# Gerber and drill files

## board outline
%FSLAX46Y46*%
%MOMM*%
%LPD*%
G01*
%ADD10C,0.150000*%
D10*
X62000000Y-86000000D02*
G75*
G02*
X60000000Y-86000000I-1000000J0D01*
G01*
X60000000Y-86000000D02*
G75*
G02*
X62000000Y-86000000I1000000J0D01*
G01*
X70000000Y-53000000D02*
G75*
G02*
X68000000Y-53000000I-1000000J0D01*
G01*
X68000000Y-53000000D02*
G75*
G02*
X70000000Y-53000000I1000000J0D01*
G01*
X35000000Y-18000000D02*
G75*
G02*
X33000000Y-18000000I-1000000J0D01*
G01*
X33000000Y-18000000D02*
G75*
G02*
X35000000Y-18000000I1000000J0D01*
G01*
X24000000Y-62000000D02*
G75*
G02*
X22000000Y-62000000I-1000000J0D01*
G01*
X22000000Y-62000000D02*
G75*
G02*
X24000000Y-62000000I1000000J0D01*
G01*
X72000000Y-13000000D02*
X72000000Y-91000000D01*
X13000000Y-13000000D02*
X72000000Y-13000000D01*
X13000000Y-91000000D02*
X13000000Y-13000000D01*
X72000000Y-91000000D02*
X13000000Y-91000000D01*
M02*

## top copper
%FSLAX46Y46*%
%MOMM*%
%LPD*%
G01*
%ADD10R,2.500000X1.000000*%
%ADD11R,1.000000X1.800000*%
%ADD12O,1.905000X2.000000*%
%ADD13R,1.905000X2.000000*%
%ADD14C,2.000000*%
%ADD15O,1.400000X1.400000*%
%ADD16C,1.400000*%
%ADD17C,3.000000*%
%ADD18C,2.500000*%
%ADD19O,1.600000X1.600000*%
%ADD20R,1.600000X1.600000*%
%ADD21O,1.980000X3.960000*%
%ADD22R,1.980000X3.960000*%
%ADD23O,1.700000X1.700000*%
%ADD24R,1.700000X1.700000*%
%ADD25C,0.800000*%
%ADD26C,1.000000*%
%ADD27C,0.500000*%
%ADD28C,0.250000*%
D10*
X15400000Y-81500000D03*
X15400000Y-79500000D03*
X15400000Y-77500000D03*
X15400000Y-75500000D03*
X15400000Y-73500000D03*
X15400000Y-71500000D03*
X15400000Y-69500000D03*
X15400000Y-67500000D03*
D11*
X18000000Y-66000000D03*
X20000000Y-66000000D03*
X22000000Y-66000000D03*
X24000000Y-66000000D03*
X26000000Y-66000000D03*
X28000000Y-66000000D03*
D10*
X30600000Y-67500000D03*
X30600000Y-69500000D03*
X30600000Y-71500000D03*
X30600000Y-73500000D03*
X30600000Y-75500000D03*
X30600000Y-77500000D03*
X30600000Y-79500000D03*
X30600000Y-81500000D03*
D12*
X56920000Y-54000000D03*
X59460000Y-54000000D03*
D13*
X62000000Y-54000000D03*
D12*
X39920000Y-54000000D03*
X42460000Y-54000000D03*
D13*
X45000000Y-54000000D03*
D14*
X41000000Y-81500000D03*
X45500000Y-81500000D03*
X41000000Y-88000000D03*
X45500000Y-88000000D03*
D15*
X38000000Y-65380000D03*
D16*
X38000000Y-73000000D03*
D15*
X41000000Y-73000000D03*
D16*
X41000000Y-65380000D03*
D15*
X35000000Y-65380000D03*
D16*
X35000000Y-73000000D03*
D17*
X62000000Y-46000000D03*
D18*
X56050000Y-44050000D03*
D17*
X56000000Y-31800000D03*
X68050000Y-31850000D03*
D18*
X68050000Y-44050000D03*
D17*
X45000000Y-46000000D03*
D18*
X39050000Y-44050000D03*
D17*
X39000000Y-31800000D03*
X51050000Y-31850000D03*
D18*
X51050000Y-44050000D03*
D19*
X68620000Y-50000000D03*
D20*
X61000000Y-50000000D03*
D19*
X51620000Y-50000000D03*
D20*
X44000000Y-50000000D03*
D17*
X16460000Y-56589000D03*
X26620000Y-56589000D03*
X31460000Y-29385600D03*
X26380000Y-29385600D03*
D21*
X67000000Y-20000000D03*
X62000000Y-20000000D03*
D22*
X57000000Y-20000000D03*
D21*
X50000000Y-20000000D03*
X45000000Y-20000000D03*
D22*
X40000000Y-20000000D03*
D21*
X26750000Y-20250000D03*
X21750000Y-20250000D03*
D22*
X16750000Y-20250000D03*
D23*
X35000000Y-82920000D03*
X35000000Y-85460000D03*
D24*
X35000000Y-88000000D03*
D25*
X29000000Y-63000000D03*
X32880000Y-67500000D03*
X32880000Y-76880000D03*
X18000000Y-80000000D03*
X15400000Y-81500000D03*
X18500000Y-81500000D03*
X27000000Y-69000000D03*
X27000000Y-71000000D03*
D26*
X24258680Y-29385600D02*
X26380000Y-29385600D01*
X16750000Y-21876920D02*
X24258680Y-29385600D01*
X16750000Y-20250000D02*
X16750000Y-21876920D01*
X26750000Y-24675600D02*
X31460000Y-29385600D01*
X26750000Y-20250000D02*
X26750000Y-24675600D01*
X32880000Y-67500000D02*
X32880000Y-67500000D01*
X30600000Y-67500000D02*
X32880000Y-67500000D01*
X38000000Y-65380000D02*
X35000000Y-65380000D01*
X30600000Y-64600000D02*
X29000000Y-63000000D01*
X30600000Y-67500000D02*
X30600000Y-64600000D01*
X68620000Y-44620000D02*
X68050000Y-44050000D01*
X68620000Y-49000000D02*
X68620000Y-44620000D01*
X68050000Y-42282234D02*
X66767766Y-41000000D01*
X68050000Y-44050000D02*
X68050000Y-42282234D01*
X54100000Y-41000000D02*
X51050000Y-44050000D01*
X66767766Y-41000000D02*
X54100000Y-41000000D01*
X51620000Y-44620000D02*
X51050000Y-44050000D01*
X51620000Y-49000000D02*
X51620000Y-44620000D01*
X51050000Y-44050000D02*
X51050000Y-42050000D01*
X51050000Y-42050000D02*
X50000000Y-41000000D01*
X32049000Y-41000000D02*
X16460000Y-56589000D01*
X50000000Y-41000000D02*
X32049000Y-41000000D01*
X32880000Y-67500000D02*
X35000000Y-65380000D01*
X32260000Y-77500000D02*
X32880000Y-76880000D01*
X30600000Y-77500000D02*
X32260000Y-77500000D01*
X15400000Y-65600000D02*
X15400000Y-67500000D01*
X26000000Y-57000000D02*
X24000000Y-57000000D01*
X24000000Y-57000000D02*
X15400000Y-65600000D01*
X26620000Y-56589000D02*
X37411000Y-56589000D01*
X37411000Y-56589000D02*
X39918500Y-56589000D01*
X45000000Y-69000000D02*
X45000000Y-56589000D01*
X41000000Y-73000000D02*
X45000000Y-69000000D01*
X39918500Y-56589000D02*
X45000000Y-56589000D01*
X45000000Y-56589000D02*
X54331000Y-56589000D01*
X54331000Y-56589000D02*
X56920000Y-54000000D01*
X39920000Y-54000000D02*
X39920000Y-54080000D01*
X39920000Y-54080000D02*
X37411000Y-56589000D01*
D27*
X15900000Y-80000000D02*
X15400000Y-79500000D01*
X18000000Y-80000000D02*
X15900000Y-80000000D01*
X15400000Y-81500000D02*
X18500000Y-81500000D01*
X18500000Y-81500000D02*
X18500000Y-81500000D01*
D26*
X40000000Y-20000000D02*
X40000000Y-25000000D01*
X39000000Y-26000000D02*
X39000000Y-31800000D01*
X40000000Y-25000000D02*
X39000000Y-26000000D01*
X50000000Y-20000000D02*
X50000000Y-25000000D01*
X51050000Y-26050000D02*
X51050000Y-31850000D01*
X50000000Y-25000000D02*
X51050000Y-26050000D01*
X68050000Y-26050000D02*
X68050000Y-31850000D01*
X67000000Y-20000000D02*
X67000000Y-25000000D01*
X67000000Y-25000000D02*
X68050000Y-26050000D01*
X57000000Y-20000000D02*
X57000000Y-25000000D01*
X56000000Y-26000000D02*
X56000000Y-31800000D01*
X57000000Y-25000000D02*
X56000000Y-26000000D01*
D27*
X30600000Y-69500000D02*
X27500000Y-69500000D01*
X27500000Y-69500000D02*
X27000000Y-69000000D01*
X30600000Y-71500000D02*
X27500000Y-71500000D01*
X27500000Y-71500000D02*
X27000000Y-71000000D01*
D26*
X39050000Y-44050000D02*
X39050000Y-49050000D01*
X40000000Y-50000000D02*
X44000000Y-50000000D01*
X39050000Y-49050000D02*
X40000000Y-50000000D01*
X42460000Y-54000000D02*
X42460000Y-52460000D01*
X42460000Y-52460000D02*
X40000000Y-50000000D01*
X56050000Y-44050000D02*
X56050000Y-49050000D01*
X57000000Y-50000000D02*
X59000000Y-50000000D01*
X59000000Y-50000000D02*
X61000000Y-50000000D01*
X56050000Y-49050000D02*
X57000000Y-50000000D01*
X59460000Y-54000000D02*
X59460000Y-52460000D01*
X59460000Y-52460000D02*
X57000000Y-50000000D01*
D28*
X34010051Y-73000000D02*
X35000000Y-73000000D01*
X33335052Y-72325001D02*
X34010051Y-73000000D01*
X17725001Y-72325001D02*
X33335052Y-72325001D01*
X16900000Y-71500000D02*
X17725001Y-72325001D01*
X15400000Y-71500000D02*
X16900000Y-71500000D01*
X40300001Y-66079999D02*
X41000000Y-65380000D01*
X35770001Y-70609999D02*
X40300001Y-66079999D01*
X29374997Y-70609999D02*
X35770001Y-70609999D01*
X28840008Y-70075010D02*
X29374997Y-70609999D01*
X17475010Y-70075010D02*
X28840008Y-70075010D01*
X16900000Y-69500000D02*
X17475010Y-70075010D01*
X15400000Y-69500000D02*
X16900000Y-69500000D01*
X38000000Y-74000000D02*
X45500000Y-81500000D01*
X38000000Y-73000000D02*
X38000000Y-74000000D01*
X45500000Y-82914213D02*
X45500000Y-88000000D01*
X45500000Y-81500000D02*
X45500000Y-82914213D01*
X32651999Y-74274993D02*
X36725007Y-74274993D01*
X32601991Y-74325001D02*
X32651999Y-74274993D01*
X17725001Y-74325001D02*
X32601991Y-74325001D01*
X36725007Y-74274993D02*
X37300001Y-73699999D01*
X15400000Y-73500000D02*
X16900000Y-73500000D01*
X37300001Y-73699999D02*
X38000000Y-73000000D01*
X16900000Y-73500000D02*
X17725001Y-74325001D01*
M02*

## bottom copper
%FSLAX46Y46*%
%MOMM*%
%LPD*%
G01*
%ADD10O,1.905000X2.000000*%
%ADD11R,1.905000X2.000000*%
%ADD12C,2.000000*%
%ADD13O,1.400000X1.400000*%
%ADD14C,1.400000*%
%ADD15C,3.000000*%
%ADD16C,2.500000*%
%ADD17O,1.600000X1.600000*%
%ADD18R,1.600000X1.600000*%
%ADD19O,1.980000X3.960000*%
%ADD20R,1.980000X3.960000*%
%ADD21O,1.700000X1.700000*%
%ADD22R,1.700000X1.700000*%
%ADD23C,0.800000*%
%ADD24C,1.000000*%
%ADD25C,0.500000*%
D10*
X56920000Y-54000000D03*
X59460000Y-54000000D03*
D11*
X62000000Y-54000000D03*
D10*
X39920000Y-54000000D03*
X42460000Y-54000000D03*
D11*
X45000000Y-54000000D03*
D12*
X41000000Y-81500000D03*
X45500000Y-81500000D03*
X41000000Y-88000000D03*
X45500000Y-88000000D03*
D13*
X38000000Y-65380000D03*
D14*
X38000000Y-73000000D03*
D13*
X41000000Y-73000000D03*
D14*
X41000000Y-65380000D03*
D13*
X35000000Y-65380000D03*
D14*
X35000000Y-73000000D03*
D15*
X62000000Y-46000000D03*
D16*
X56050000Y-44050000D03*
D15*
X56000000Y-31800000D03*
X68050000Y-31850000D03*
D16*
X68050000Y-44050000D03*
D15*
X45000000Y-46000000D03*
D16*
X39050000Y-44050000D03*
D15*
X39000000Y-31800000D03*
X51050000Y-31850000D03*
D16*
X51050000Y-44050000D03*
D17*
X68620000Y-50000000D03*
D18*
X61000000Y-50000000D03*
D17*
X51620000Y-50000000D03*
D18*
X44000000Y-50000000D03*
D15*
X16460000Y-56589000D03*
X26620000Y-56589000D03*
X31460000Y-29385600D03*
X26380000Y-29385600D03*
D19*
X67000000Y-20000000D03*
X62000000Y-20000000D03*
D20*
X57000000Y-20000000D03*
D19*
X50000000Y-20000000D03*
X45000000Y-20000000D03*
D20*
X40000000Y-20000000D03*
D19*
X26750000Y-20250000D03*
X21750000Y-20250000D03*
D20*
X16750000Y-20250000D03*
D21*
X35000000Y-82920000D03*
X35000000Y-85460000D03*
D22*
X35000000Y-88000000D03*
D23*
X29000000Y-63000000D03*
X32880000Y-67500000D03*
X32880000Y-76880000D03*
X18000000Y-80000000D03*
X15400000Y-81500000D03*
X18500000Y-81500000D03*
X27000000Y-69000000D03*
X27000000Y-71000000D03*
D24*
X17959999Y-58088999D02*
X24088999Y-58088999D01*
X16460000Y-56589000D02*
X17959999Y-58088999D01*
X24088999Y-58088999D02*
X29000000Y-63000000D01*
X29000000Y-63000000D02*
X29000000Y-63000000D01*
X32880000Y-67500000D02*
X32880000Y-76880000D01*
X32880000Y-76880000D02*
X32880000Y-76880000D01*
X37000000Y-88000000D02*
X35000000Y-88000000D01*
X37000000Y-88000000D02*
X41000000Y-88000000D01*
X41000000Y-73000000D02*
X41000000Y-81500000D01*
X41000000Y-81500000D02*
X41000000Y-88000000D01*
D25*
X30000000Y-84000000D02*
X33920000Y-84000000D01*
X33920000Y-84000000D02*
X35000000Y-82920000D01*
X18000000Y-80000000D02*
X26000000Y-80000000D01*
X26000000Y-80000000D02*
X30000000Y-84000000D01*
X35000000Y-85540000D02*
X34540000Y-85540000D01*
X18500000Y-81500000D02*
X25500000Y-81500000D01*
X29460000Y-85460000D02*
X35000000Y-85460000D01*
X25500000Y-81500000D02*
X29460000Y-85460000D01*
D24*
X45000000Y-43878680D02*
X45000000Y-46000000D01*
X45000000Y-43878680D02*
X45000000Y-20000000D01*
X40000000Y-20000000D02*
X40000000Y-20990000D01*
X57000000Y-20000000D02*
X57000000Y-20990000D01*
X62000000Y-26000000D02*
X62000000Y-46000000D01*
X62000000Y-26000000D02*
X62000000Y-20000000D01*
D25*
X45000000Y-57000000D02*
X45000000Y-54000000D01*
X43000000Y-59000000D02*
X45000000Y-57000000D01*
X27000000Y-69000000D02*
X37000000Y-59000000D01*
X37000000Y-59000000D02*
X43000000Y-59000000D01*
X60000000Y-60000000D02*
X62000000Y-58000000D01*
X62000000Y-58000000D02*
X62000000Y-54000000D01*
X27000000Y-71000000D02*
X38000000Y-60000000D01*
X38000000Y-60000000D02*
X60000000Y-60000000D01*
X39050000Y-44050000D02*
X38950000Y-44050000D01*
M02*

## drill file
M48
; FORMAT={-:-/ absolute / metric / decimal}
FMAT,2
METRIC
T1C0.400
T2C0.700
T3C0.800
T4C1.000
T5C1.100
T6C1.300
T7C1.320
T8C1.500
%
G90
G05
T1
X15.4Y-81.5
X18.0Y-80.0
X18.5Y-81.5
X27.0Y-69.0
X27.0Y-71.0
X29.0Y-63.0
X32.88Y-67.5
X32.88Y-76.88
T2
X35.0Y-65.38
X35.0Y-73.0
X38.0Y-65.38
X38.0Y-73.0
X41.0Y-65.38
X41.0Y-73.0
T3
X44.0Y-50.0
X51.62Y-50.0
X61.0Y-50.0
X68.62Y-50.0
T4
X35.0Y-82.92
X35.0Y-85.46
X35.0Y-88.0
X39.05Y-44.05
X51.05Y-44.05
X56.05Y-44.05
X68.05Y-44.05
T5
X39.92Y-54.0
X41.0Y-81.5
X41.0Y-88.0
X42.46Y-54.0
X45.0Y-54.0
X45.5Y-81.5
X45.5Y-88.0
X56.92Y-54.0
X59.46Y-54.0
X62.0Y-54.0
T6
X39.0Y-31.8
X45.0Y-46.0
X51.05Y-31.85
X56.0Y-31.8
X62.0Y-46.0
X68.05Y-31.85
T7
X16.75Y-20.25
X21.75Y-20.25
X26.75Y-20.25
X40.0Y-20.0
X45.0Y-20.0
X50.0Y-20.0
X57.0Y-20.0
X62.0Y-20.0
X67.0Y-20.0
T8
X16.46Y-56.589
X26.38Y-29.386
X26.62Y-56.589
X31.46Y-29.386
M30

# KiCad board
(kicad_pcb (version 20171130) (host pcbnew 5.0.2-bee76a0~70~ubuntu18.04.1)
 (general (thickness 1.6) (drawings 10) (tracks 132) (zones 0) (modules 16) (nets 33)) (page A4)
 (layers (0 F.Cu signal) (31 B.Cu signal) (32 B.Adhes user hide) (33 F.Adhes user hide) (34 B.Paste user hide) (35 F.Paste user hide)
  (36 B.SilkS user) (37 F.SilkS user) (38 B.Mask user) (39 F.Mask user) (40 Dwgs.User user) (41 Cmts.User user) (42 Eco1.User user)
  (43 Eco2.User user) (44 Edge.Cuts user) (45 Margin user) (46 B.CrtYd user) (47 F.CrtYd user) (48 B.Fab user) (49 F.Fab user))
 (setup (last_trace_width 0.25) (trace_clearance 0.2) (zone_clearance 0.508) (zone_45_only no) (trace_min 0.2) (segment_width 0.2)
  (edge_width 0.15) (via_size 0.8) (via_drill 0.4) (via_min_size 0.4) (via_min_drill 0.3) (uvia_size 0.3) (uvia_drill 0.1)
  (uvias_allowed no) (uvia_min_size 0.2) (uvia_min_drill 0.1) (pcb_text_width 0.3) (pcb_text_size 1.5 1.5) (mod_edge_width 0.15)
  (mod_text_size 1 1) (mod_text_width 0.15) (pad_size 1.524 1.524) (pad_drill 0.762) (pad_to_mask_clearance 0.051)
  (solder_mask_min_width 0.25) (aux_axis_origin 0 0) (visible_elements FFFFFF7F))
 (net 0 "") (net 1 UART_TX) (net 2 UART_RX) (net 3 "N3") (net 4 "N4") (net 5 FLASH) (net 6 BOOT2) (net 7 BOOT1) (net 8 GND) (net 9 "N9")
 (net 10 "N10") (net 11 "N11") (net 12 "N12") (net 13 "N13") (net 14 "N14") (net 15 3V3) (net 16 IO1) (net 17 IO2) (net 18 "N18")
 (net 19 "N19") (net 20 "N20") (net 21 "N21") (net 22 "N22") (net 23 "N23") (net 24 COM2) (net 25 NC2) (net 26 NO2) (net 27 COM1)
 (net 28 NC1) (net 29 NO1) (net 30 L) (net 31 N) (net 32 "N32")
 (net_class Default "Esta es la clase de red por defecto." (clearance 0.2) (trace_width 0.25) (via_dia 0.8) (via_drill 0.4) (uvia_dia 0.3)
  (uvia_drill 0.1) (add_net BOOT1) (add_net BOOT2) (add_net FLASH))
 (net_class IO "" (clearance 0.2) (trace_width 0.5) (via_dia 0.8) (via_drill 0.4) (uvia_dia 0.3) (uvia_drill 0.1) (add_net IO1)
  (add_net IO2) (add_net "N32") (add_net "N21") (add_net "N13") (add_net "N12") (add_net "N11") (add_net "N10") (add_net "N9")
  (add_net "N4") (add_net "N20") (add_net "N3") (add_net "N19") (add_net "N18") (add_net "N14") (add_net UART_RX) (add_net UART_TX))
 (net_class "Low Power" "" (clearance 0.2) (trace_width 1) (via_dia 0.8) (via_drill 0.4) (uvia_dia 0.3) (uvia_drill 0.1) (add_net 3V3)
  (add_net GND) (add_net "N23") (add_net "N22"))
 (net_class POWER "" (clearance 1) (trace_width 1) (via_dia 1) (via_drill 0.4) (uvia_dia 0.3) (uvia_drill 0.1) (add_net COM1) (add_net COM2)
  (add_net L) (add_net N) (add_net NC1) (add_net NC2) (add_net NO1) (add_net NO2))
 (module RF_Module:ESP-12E (layer F.Cu) (at 23 78 180)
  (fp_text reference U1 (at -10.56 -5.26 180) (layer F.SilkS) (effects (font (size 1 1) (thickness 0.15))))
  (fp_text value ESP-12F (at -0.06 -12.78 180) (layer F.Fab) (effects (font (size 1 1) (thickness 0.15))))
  (pad 22 smd rect (at 7.6 -3.5 180) (size 2.5 1) (layers F.Cu F.Paste F.Mask) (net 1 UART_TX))
  (pad 21 smd rect (at 7.6 -1.5 180) (size 2.5 1) (layers F.Cu F.Paste F.Mask) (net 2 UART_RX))
  (pad 20 smd rect (at 7.6 0.5 180) (size 2.5 1) (layers F.Cu F.Paste F.Mask) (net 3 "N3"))
  (pad 19 smd rect (at 7.6 2.5 180) (size 2.5 1) (layers F.Cu F.Paste F.Mask) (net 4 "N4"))
  (pad 18 smd rect (at 7.6 4.5 180) (size 2.5 1) (layers F.Cu F.Paste F.Mask) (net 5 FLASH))
  (pad 17 smd rect (at 7.6 6.5 180) (size 2.5 1) (layers F.Cu F.Paste F.Mask) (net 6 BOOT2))
  (pad 16 smd rect (at 7.6 8.5 180) (size 2.5 1) (layers F.Cu F.Paste F.Mask) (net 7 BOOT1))
  (pad 15 smd rect (at 7.6 10.5 180) (size 2.5 1) (layers F.Cu F.Paste F.Mask) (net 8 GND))
  (pad 14 smd rect (at 5 12 180) (size 1 1.8) (layers F.Cu F.Paste F.Mask) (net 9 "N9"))
  (pad 13 smd rect (at 3 12 180) (size 1 1.8) (layers F.Cu F.Paste F.Mask) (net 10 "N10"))
  (pad 12 smd rect (at 1 12 180) (size 1 1.8) (layers F.Cu F.Paste F.Mask) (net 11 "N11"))
  (pad 11 smd rect (at -1 12 180) (size 1 1.8) (layers F.Cu F.Paste F.Mask) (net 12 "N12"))
  (pad 10 smd rect (at -3 12 180) (size 1 1.8) (layers F.Cu F.Paste F.Mask) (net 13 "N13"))
  (pad 9 smd rect (at -5 12 180) (size 1 1.8) (layers F.Cu F.Paste F.Mask) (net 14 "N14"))
  (pad 8 smd rect (at -7.6 10.5 180) (size 2.5 1) (layers F.Cu F.Paste F.Mask) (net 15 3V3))
  (pad 7 smd rect (at -7.6 8.5 180) (size 2.5 1) (layers F.Cu F.Paste F.Mask) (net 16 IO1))
  (pad 6 smd rect (at -7.6 6.5 180) (size 2.5 1) (layers F.Cu F.Paste F.Mask) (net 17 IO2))
  (pad 5 smd rect (at -7.6 4.5 180) (size 2.5 1) (layers F.Cu F.Paste F.Mask) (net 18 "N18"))
  (pad 4 smd rect (at -7.6 2.5 180) (size 2.5 1) (layers F.Cu F.Paste F.Mask) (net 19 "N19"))
  (pad 3 smd rect (at -7.6 0.5 180) (size 2.5 1) (layers F.Cu F.Paste F.Mask) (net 15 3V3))
  (pad 2 smd rect (at -7.6 -1.5 180) (size 2.5 1) (layers F.Cu F.Paste F.Mask) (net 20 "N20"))
  (pad 1 smd rect (at -7.6 -3.5 180) (size 2.5 1) (layers F.Cu F.Paste F.Mask) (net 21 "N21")))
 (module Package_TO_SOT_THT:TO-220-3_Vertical (layer F.Cu) (at 62 54 180)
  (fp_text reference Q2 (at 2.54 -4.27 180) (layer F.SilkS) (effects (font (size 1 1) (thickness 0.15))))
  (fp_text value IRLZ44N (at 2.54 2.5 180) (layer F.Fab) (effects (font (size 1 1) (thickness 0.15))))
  (pad 3 thru_hole oval (at 5.08 0 180) (size 1.905 2) (drill 1.1) (layers *.Cu *.Mask) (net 8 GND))
  (pad 2 thru_hole oval (at 2.54 0 180) (size 1.905 2) (drill 1.1) (layers *.Cu *.Mask) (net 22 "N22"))
  (pad 1 thru_hole rect (at 0 0 180) (size 1.905 2) (drill 1.1) (layers *.Cu *.Mask) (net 17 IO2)))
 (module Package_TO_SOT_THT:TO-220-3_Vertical (layer F.Cu) (at 45 54 180)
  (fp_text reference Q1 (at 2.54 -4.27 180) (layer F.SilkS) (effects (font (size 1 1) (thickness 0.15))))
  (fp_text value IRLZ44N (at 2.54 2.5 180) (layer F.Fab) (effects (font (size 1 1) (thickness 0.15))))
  (pad 3 thru_hole oval (at 5.08 0 180) (size 1.905 2) (drill 1.1) (layers *.Cu *.Mask) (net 8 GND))
  (pad 2 thru_hole oval (at 2.54 0 180) (size 1.905 2) (drill 1.1) (layers *.Cu *.Mask) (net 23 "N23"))
  (pad 1 thru_hole rect (at 0 0 180) (size 1.905 2) (drill 1.1) (layers *.Cu *.Mask) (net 16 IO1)))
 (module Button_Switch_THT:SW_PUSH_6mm (layer F.Cu) (at 41 88 90)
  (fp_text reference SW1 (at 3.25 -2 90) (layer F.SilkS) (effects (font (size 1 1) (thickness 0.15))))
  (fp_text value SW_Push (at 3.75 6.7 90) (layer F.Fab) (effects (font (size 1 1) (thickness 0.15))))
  (pad 1 thru_hole circle (at 6.5 0 180) (size 2 2) (drill 1.1) (layers *.Cu *.Mask) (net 8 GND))
  (pad 2 thru_hole circle (at 6.5 4.5 180) (size 2 2) (drill 1.1) (layers *.Cu *.Mask) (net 5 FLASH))
  (pad 1 thru_hole circle (at 0 0 180) (size 2 2) (drill 1.1) (layers *.Cu *.Mask) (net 8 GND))
  (pad 2 thru_hole circle (at 0 4.5 180) (size 2 2) (drill 1.1) (layers *.Cu *.Mask) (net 5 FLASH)))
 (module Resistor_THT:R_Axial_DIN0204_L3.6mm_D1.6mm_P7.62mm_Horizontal (layer F.Cu) (at 38 73 90)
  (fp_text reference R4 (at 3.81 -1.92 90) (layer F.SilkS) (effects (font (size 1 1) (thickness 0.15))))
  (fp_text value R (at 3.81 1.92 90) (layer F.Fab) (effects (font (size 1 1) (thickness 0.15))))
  (pad 2 thru_hole oval (at 7.62 0 90) (size 1.4 1.4) (drill 0.7) (layers *.Cu *.Mask) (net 15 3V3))
  (pad 1 thru_hole circle (at 0 0 90) (size 1.4 1.4) (drill 0.7) (layers *.Cu *.Mask) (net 5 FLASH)))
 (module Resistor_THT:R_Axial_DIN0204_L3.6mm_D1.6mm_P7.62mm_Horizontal (layer F.Cu) (at 41 65.38 270)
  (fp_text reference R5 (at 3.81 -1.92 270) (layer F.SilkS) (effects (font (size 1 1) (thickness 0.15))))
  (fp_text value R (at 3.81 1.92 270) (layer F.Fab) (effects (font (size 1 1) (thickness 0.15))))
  (pad 2 thru_hole oval (at 7.62 0 270) (size 1.4 1.4) (drill 0.7) (layers *.Cu *.Mask) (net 8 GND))
  (pad 1 thru_hole circle (at 0 0 270) (size 1.4 1.4) (drill 0.7) (layers *.Cu *.Mask) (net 7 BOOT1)))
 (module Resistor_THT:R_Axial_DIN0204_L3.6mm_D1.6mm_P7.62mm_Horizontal (layer F.Cu) (at 35 73 90)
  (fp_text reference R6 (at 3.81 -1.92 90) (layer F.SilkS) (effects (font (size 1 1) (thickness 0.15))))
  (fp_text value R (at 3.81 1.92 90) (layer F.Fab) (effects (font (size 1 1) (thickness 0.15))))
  (pad 2 thru_hole oval (at 7.62 0 90) (size 1.4 1.4) (drill 0.7) (layers *.Cu *.Mask) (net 15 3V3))
  (pad 1 thru_hole circle (at 0 0 90) (size 1.4 1.4) (drill 0.7) (layers *.Cu *.Mask) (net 6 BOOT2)))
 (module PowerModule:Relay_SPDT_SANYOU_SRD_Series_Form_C (layer F.Cu) (at 62 46 90)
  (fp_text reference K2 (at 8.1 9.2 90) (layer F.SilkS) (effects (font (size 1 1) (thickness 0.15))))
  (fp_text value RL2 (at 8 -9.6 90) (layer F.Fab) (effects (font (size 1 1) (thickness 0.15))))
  (pad 5 thru_hole circle (at 0 0 180) (size 3 3) (drill 1.3) (layers *.Cu *.Mask) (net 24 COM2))
  (pad 4 thru_hole circle (at 1.95 -5.95 180) (size 2.5 2.5) (drill 1) (layers *.Cu *.Mask) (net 22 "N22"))
  (pad 2 thru_hole circle (at 14.2 -6 180) (size 3 3) (drill 1.3) (layers *.Cu *.Mask) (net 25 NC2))
  (pad 1 thru_hole circle (at 14.15 6.05 180) (size 3 3) (drill 1.3) (layers *.Cu *.Mask) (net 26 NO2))
  (pad 3 thru_hole circle (at 1.95 6.05 180) (size 2.5 2.5) (drill 1) (layers *.Cu *.Mask) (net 15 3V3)))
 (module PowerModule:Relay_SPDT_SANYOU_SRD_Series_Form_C (layer F.Cu) (at 45 46 90)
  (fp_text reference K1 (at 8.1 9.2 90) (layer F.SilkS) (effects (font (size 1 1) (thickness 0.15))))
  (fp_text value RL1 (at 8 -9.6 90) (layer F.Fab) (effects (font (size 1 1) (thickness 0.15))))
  (pad 5 thru_hole circle (at 0 0 180) (size 3 3) (drill 1.3) (layers *.Cu *.Mask) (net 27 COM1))
  (pad 4 thru_hole circle (at 1.95 -5.95 180) (size 2.5 2.5) (drill 1) (layers *.Cu *.Mask) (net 23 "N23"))
  (pad 2 thru_hole circle (at 14.2 -6 180) (size 3 3) (drill 1.3) (layers *.Cu *.Mask) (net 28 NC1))
  (pad 1 thru_hole circle (at 14.15 6.05 180) (size 3 3) (drill 1.3) (layers *.Cu *.Mask) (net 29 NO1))
  (pad 3 thru_hole circle (at 1.95 6.05 180) (size 2.5 2.5) (drill 1) (layers *.Cu *.Mask) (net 15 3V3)))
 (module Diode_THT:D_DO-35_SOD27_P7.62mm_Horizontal (layer F.Cu) (at 61 50)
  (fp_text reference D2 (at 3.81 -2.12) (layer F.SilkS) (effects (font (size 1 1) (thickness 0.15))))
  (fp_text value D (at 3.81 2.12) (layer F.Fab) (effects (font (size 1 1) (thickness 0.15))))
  (pad 2 thru_hole oval (at 7.62 0) (size 1.6 1.6) (drill 0.8) (layers *.Cu *.Mask) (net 15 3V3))
  (pad 1 thru_hole rect (at 0 0) (size 1.6 1.6) (drill 0.8) (layers *.Cu *.Mask) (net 22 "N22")))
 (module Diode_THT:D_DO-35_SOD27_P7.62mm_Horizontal (layer F.Cu) (at 44 50)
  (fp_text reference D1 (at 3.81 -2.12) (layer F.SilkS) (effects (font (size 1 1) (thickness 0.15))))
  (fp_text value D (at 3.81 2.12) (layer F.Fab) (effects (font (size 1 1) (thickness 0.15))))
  (pad 2 thru_hole oval (at 7.62 0) (size 1.6 1.6) (drill 0.8) (layers *.Cu *.Mask) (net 15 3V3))
  (pad 1 thru_hole rect (at 0 0) (size 1.6 1.6) (drill 0.8) (layers *.Cu *.Mask) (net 23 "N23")))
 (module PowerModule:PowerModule (layer F.Cu) (at 24 43 270)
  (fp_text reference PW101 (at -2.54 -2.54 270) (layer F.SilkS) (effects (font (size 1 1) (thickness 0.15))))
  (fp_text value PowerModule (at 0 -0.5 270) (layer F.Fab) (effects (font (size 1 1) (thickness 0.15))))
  (pad 4 thru_hole circle (at 13.589 7.54 270) (size 3 3) (drill 1.5) (layers *.Cu *.Mask) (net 15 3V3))
  (pad 3 thru_hole circle (at 13.589 -2.62 270) (size 3 3) (drill 1.5) (layers *.Cu *.Mask) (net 8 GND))
  (pad 2 thru_hole circle (at -13.6144 -7.46 270) (size 3 3) (drill 1.5) (layers *.Cu *.Mask) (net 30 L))
  (pad 1 thru_hole circle (at -13.6144 -2.38 270) (size 3 3) (drill 1.5) (layers *.Cu *.Mask) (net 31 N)))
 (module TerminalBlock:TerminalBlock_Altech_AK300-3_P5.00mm (layer F.Cu) (at 57 20)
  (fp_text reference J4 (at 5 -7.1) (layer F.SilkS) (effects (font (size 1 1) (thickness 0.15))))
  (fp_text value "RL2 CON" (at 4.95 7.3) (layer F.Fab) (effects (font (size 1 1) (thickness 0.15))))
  (pad 3 thru_hole oval (at 10 0) (size 1.98 3.96) (drill 1.32) (layers *.Cu *.Mask) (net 26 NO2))
  (pad 2 thru_hole oval (at 5 0) (size 1.98 3.96) (drill 1.32) (layers *.Cu *.Mask) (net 24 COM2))
  (pad 1 thru_hole rect (at 0 0) (size 1.98 3.96) (drill 1.32) (layers *.Cu *.Mask) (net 25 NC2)))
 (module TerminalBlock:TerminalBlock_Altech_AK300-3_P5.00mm (layer F.Cu) (at 40 20)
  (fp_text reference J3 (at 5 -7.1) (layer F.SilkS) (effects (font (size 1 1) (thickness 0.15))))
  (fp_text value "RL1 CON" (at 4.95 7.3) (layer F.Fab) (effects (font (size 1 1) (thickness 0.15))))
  (pad 3 thru_hole oval (at 10 0) (size 1.98 3.96) (drill 1.32) (layers *.Cu *.Mask) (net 29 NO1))
  (pad 2 thru_hole oval (at 5 0) (size 1.98 3.96) (drill 1.32) (layers *.Cu *.Mask) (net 27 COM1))
  (pad 1 thru_hole rect (at 0 0) (size 1.98 3.96) (drill 1.32) (layers *.Cu *.Mask) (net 28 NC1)))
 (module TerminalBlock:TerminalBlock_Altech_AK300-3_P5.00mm (layer F.Cu) (at 16.75 20.25)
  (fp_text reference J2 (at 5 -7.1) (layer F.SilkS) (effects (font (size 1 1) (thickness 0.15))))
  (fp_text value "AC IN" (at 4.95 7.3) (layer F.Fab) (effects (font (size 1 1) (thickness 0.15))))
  (pad 3 thru_hole oval (at 10 0) (size 1.98 3.96) (drill 1.32) (layers *.Cu *.Mask) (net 30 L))
  (pad 2 thru_hole oval (at 5 0) (size 1.98 3.96) (drill 1.32) (layers *.Cu *.Mask) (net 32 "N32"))
  (pad 1 thru_hole rect (at 0 0) (size 1.98 3.96) (drill 1.32) (layers *.Cu *.Mask) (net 31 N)))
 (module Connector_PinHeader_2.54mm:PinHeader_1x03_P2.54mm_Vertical (layer F.Cu) (at 35 88 180)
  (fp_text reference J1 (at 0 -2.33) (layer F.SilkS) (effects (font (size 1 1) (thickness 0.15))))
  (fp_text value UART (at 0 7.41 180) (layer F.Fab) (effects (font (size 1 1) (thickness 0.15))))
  (pad 3 thru_hole oval (at 0 5.08 180) (size 1.7 1.7) (drill 1) (layers *.Cu *.Mask) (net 2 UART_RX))
  (pad 2 thru_hole oval (at 0 2.54 180) (size 1.7 1.7) (drill 1) (layers *.Cu *.Mask) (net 1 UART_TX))
  (pad 1 thru_hole rect (at 0 0 180) (size 1.7 1.7) (drill 1) (layers *.Cu *.Mask) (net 8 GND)))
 (gr_circle (center 61 86) (end 62 86) (layer Edge.Cuts) (width 0.15))
 (gr_circle (center 69 53) (end 69 54) (layer Edge.Cuts) (width 0.15))
 (gr_circle (center 34 18) (end 34 19) (layer Edge.Cuts) (width 0.15))
 (gr_circle (center 23 62) (end 24 62) (layer Edge.Cuts) (width 0.15))
 (gr_line (start 72 13) (end 72 91) (layer Edge.Cuts) (width 0.15))
 (gr_line (start 13 13) (end 72 13) (layer Edge.Cuts) (width 0.15))
 (gr_line (start 13 91) (end 13 13) (layer Edge.Cuts) (width 0.15))
 (gr_line (start 72 91) (end 13 91) (layer Edge.Cuts) (width 0.15))
 (segment (start 24.25868 29.3856) (end 26.38 29.3856) (width 1) (layer F.Cu) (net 31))
 (segment (start 16.75 21.87692) (end 24.25868 29.3856) (width 1) (layer F.Cu) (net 31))
 (segment (start 16.75 20.25) (end 16.75 21.87692) (width 1) (layer F.Cu) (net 31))
 (segment (start 26.75 24.6756) (end 31.46 29.3856) (width 1) (layer F.Cu) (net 30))
 (segment (start 26.75 20.25) (end 26.75 24.6756) (width 1) (layer F.Cu) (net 30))
 (segment (start 32.88 67.5) (end 32.88 67.5) (width 1) (layer F.Cu) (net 15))
 (segment (start 30.6 67.5) (end 32.88 67.5) (width 1) (layer F.Cu) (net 15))
 (segment (start 38 65.38) (end 35 65.38) (width 1) (layer F.Cu) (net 15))
 (segment (start 17.959999 58.088999) (end 24.088999 58.088999) (width 1) (layer B.Cu) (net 15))
 (segment (start 16.46 56.589) (end 17.959999 58.088999) (width 1) (layer B.Cu) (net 15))
 (segment (start 24.088999 58.088999) (end 29 63) (width 1) (layer B.Cu) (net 15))
 (segment (start 29 63) (end 29 63) (width 1) (layer B.Cu) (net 15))
 (via (at 29 63) (size 0.8) (drill 0.4) (layers F.Cu B.Cu) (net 15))
 (segment (start 30.6 64.6) (end 29 63) (width 1) (layer F.Cu) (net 15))
 (segment (start 30.6 67.5) (end 30.6 64.6) (width 1) (layer F.Cu) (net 15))
 (segment (start 68.62 44.62) (end 68.05 44.05) (width 1) (layer F.Cu) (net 15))
 (segment (start 68.62 49) (end 68.62 44.62) (width 1) (layer F.Cu) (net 15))
 (segment (start 68.05 42.282234) (end 66.767766 41) (width 1) (layer F.Cu) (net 15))
 (segment (start 68.05 44.05) (end 68.05 42.282234) (width 1) (layer F.Cu) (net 15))
 (segment (start 54.1 41) (end 51.05 44.05) (width 1) (layer F.Cu) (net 15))
 (segment (start 66.767766 41) (end 54.1 41) (width 1) (layer F.Cu) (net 15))
 (segment (start 51.62 44.62) (end 51.05 44.05) (width 1) (layer F.Cu) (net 15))
 (segment (start 51.62 49) (end 51.62 44.62) (width 1) (layer F.Cu) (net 15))
 (segment (start 51.05 44.05) (end 51.05 42.05) (width 1) (layer F.Cu) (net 15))
 (segment (start 51.05 42.05) (end 50 41) (width 1) (layer F.Cu) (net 15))
 (segment (start 32.049 41) (end 16.46 56.589) (width 1) (layer F.Cu) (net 15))
 (segment (start 50 41) (end 32.049 41) (width 1) (layer F.Cu) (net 15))
 (segment (start 32.88 67.5) (end 35 65.38) (width 1) (layer F.Cu) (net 15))
 (via (at 32.88 67.5) (size 0.8) (drill 0.4) (layers F.Cu B.Cu) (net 15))
 (segment (start 32.88 67.5) (end 32.88 76.88) (width 1) (layer B.Cu) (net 15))
 (segment (start 32.88 76.88) (end 32.88 76.88) (width 1) (layer B.Cu) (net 15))
 (via (at 32.88 76.88) (size 0.8) (drill 0.4) (layers F.Cu B.Cu) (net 15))
 (segment (start 32.26 77.5) (end 32.88 76.88) (width 1) (layer F.Cu) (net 15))
 (segment (start 30.6 77.5) (end 32.26 77.5) (width 1) (layer F.Cu) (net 15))
 (segment (start 15.4 65.6) (end 15.4 67.5) (width 1) (layer F.Cu) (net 8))
 (segment (start 26 57) (end 24 57) (width 1) (layer F.Cu) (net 8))
 (segment (start 24 57) (end 15.4 65.6) (width 1) (layer F.Cu) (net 8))
 (segment (start 37 88) (end 35 88) (width 1) (layer B.Cu) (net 8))
 (segment (start 37 88) (end 41 88) (width 1) (layer B.Cu) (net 8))
 (segment (start 41 73) (end 41 81.5) (width 1) (layer B.Cu) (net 8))
 (segment (start 41 81.5) (end 41 88) (width 1) (layer B.Cu) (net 8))
 (segment (start 26.62 56.589) (end 37.411 56.589) (width 1) (layer F.Cu) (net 8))
 (segment (start 37.411 56.589) (end 39.9185 56.589) (width 1) (layer F.Cu) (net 8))
 (segment (start 45 69) (end 45 56.589) (width 1) (layer F.Cu) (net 8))
 (segment (start 41 73) (end 45 69) (width 1) (layer F.Cu) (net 8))
 (segment (start 39.9185 56.589) (end 45 56.589) (width 1) (layer F.Cu) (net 8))
 (segment (start 45 56.589) (end 54.331 56.589) (width 1) (layer F.Cu) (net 8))
 (segment (start 54.331 56.589) (end 56.92 54) (width 1) (layer F.Cu) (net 8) (status 800000))
 (segment (start 39.92 54) (end 39.92 54.08) (width 1) (layer F.Cu) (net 8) (status C00000))
 (segment (start 39.92 54.08) (end 37.411 56.589) (width 1) (layer F.Cu) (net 8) (status 400000))
 (via (at 18 80) (size 0.8) (drill 0.4) (layers F.Cu B.Cu) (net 2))
 (segment (start 15.9 80) (end 15.4 79.5) (width 0.5) (layer F.Cu) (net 2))
 (segment (start 18 80) (end 15.9 80) (width 0.5) (layer F.Cu) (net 2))
 (segment (start 30 84) (end 33.92 84) (width 0.5) (layer B.Cu) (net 2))
 (segment (start 33.92 84) (end 35 82.92) (width 0.5) (layer B.Cu) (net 2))
 (segment (start 18 80) (end 26 80) (width 0.5) (layer B.Cu) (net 2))
 (segment (start 26 80) (end 30 84) (width 0.5) (layer B.Cu) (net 2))
 (segment (start 35 85.54) (end 34.54 85.54) (width 0.5) (layer B.Cu) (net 1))
 (via (at 15.4 81.5) (size 0.8) (drill 0.4) (layers F.Cu B.Cu) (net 1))
 (segment (start 15.4 81.5) (end 18.5 81.5) (width 0.5) (layer F.Cu) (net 1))
 (segment (start 18.5 81.5) (end 18.5 81.5) (width 0.5) (layer F.Cu) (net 1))
 (via (at 18.5 81.5) (size 0.8) (drill 0.4) (layers F.Cu B.Cu) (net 1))
 (segment (start 18.5 81.5) (end 25.5 81.5) (width 0.5) (layer B.Cu) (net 1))
 (segment (start 29.46 85.46) (end 35 85.46) (width 0.5) (layer B.Cu) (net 1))
 (segment (start 25.5 81.5) (end 29.46 85.46) (width 0.5) (layer B.Cu) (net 1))
 (segment (start 45 43.87868) (end 45 46) (width 1) (layer B.Cu) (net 27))
 (segment (start 45 43.87868) (end 45 20) (width 1) (layer B.Cu) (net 27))
 (segment (start 40 20) (end 40 20.99) (width 1) (layer B.Cu) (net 28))
 (segment (start 40 20) (end 40 25) (width 1) (layer F.Cu) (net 28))
 (segment (start 39 26) (end 39 31.8) (width 1) (layer F.Cu) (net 28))
 (segment (start 40 25) (end 39 26) (width 1) (layer F.Cu) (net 28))
 (segment (start 50 20) (end 50 25) (width 1) (layer F.Cu) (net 29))
 (segment (start 51.05 26.05) (end 51.05 31.85) (width 1) (layer F.Cu) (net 29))
 (segment (start 50 25) (end 51.05 26.05) (width 1) (layer F.Cu) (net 29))
 (segment (start 68.05 26.05) (end 68.05 31.85) (width 1) (layer F.Cu) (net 26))
 (segment (start 67 20) (end 67 25) (width 1) (layer F.Cu) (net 26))
 (segment (start 67 25) (end 68.05 26.05) (width 1) (layer F.Cu) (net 26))
 (segment (start 57 20) (end 57 20.99) (width 1) (layer B.Cu) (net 25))
 (segment (start 57 20) (end 57 25) (width 1) (layer F.Cu) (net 25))
 (segment (start 56 26) (end 56 31.8) (width 1) (layer F.Cu) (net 25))
 (segment (start 57 25) (end 56 26) (width 1) (layer F.Cu) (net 25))
 (segment (start 62 26) (end 62 46) (width 1) (layer B.Cu) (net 24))
 (segment (start 62 26) (end 62 20) (width 1) (layer B.Cu) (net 24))
 (segment (start 30.6 69.5) (end 27.5 69.5) (width 0.5) (layer F.Cu) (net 16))
 (segment (start 27.5 69.5) (end 27 69) (width 0.5) (layer F.Cu) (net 16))
 (via (at 27 69) (size 0.8) (drill 0.4) (layers F.Cu B.Cu) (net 16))
 (segment (start 45 57) (end 45 54) (width 0.5) (layer B.Cu) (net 16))
 (segment (start 43 59) (end 45 57) (width 0.5) (layer B.Cu) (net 16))
 (segment (start 27 69) (end 37 59) (width 0.5) (layer B.Cu) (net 16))
 (segment (start 37 59) (end 43 59) (width 0.5) (layer B.Cu) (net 16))
 (via (at 27 71) (size 0.8) (drill 0.4) (layers F.Cu B.Cu) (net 17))
 (segment (start 30.6 71.5) (end 27.5 71.5) (width 0.5) (layer F.Cu) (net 17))
 (segment (start 27.5 71.5) (end 27 71) (width 0.5) (layer F.Cu) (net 17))
 (segment (start 60 60) (end 62 58) (width 0.5) (layer B.Cu) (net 17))
 (segment (start 62 58) (end 62 54) (width 0.5) (layer B.Cu) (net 17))
 (segment (start 27 71) (end 38 60) (width 0.5) (layer B.Cu) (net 17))
 (segment (start 38 60) (end 60 60) (width 0.5) (layer B.Cu) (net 17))
 (segment (start 39.05 44.05) (end 38.95 44.05) (width 0.5) (layer B.Cu) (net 23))
 (segment (start 39.05 44.05) (end 39.05 49.05) (width 1) (layer F.Cu) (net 23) (status 400000))
 (segment (start 40 50) (end 44 50) (width 1) (layer F.Cu) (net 23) (status 800000))
 (segment (start 39.05 49.05) (end 40 50) (width 1) (layer F.Cu) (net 23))
 (segment (start 42.46 54) (end 42.46 52.46) (width 1) (layer F.Cu) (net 23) (status 400000))
 (segment (start 42.46 52.46) (end 40 50) (width 1) (layer F.Cu) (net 23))
 (segment (start 56.05 44.05) (end 56.05 49.05) (width 1) (layer F.Cu) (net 22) (status 400000))
 (segment (start 57 50) (end 59 50) (width 1) (layer F.Cu) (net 22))
 (segment (start 59 50) (end 61 50) (width 1) (layer F.Cu) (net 22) (status 800000))
 (segment (start 56.05 49.05) (end 57 50) (width 1) (layer F.Cu) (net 22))
 (segment (start 59.46 54) (end 59.46 52.46) (width 1) (layer F.Cu) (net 22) (status 400000))
 (segment (start 59.46 52.46) (end 57 50) (width 1) (layer F.Cu) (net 22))
 (segment (start 34.010051 73) (end 35 73) (width 0.25) (layer F.Cu) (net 6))
 (segment (start 33.335052 72.325001) (end 34.010051 73) (width 0.25) (layer F.Cu) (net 6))
 (segment (start 17.725001 72.325001) (end 33.335052 72.325001) (width 0.25) (layer F.Cu) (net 6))
 (segment (start 16.9 71.5) (end 17.725001 72.325001) (width 0.25) (layer F.Cu) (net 6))
 (segment (start 15.4 71.5) (end 16.9 71.5) (width 0.25) (layer F.Cu) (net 6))
 (segment (start 40.300001 66.079999) (end 41 65.38) (width 0.25) (layer F.Cu) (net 7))
 (segment (start 35.770001 70.609999) (end 40.300001 66.079999) (width 0.25) (layer F.Cu) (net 7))
 (segment (start 29.374997 70.609999) (end 35.770001 70.609999) (width 0.25) (layer F.Cu) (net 7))
 (segment (start 28.840008 70.07501) (end 29.374997 70.609999) (width 0.25) (layer F.Cu) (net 7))
 (segment (start 17.47501 70.07501) (end 28.840008 70.07501) (width 0.25) (layer F.Cu) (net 7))
 (segment (start 16.9 69.5) (end 17.47501 70.07501) (width 0.25) (layer F.Cu) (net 7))
 (segment (start 15.4 69.5) (end 16.9 69.5) (width 0.25) (layer F.Cu) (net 7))
 (segment (start 38 74) (end 45.5 81.5) (width 0.25) (layer F.Cu) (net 5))
 (segment (start 38 73) (end 38 74) (width 0.25) (layer F.Cu) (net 5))
 (segment (start 45.5 82.914213) (end 45.5 88) (width 0.25) (layer F.Cu) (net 5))
 (segment (start 45.5 81.5) (end 45.5 82.914213) (width 0.25) (layer F.Cu) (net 5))
 (segment (start 32.651999 74.274993) (end 36.725007 74.274993) (width 0.25) (layer F.Cu) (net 5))
 (segment (start 32.601991 74.325001) (end 32.651999 74.274993) (width 0.25) (layer F.Cu) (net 5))
 (segment (start 17.725001 74.325001) (end 32.601991 74.325001) (width 0.25) (layer F.Cu) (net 5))
 (segment (start 36.725007 74.274993) (end 37.300001 73.699999) (width 0.25) (layer F.Cu) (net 5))
 (segment (start 15.4 73.5) (end 16.9 73.5) (width 0.25) (layer F.Cu) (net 5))
 (segment (start 37.300001 73.699999) (end 38 73) (width 0.25) (layer F.Cu) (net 5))
 (segment (start 16.9 73.5) (end 17.725001 74.325001) (width 0.25) (layer F.Cu) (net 5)))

